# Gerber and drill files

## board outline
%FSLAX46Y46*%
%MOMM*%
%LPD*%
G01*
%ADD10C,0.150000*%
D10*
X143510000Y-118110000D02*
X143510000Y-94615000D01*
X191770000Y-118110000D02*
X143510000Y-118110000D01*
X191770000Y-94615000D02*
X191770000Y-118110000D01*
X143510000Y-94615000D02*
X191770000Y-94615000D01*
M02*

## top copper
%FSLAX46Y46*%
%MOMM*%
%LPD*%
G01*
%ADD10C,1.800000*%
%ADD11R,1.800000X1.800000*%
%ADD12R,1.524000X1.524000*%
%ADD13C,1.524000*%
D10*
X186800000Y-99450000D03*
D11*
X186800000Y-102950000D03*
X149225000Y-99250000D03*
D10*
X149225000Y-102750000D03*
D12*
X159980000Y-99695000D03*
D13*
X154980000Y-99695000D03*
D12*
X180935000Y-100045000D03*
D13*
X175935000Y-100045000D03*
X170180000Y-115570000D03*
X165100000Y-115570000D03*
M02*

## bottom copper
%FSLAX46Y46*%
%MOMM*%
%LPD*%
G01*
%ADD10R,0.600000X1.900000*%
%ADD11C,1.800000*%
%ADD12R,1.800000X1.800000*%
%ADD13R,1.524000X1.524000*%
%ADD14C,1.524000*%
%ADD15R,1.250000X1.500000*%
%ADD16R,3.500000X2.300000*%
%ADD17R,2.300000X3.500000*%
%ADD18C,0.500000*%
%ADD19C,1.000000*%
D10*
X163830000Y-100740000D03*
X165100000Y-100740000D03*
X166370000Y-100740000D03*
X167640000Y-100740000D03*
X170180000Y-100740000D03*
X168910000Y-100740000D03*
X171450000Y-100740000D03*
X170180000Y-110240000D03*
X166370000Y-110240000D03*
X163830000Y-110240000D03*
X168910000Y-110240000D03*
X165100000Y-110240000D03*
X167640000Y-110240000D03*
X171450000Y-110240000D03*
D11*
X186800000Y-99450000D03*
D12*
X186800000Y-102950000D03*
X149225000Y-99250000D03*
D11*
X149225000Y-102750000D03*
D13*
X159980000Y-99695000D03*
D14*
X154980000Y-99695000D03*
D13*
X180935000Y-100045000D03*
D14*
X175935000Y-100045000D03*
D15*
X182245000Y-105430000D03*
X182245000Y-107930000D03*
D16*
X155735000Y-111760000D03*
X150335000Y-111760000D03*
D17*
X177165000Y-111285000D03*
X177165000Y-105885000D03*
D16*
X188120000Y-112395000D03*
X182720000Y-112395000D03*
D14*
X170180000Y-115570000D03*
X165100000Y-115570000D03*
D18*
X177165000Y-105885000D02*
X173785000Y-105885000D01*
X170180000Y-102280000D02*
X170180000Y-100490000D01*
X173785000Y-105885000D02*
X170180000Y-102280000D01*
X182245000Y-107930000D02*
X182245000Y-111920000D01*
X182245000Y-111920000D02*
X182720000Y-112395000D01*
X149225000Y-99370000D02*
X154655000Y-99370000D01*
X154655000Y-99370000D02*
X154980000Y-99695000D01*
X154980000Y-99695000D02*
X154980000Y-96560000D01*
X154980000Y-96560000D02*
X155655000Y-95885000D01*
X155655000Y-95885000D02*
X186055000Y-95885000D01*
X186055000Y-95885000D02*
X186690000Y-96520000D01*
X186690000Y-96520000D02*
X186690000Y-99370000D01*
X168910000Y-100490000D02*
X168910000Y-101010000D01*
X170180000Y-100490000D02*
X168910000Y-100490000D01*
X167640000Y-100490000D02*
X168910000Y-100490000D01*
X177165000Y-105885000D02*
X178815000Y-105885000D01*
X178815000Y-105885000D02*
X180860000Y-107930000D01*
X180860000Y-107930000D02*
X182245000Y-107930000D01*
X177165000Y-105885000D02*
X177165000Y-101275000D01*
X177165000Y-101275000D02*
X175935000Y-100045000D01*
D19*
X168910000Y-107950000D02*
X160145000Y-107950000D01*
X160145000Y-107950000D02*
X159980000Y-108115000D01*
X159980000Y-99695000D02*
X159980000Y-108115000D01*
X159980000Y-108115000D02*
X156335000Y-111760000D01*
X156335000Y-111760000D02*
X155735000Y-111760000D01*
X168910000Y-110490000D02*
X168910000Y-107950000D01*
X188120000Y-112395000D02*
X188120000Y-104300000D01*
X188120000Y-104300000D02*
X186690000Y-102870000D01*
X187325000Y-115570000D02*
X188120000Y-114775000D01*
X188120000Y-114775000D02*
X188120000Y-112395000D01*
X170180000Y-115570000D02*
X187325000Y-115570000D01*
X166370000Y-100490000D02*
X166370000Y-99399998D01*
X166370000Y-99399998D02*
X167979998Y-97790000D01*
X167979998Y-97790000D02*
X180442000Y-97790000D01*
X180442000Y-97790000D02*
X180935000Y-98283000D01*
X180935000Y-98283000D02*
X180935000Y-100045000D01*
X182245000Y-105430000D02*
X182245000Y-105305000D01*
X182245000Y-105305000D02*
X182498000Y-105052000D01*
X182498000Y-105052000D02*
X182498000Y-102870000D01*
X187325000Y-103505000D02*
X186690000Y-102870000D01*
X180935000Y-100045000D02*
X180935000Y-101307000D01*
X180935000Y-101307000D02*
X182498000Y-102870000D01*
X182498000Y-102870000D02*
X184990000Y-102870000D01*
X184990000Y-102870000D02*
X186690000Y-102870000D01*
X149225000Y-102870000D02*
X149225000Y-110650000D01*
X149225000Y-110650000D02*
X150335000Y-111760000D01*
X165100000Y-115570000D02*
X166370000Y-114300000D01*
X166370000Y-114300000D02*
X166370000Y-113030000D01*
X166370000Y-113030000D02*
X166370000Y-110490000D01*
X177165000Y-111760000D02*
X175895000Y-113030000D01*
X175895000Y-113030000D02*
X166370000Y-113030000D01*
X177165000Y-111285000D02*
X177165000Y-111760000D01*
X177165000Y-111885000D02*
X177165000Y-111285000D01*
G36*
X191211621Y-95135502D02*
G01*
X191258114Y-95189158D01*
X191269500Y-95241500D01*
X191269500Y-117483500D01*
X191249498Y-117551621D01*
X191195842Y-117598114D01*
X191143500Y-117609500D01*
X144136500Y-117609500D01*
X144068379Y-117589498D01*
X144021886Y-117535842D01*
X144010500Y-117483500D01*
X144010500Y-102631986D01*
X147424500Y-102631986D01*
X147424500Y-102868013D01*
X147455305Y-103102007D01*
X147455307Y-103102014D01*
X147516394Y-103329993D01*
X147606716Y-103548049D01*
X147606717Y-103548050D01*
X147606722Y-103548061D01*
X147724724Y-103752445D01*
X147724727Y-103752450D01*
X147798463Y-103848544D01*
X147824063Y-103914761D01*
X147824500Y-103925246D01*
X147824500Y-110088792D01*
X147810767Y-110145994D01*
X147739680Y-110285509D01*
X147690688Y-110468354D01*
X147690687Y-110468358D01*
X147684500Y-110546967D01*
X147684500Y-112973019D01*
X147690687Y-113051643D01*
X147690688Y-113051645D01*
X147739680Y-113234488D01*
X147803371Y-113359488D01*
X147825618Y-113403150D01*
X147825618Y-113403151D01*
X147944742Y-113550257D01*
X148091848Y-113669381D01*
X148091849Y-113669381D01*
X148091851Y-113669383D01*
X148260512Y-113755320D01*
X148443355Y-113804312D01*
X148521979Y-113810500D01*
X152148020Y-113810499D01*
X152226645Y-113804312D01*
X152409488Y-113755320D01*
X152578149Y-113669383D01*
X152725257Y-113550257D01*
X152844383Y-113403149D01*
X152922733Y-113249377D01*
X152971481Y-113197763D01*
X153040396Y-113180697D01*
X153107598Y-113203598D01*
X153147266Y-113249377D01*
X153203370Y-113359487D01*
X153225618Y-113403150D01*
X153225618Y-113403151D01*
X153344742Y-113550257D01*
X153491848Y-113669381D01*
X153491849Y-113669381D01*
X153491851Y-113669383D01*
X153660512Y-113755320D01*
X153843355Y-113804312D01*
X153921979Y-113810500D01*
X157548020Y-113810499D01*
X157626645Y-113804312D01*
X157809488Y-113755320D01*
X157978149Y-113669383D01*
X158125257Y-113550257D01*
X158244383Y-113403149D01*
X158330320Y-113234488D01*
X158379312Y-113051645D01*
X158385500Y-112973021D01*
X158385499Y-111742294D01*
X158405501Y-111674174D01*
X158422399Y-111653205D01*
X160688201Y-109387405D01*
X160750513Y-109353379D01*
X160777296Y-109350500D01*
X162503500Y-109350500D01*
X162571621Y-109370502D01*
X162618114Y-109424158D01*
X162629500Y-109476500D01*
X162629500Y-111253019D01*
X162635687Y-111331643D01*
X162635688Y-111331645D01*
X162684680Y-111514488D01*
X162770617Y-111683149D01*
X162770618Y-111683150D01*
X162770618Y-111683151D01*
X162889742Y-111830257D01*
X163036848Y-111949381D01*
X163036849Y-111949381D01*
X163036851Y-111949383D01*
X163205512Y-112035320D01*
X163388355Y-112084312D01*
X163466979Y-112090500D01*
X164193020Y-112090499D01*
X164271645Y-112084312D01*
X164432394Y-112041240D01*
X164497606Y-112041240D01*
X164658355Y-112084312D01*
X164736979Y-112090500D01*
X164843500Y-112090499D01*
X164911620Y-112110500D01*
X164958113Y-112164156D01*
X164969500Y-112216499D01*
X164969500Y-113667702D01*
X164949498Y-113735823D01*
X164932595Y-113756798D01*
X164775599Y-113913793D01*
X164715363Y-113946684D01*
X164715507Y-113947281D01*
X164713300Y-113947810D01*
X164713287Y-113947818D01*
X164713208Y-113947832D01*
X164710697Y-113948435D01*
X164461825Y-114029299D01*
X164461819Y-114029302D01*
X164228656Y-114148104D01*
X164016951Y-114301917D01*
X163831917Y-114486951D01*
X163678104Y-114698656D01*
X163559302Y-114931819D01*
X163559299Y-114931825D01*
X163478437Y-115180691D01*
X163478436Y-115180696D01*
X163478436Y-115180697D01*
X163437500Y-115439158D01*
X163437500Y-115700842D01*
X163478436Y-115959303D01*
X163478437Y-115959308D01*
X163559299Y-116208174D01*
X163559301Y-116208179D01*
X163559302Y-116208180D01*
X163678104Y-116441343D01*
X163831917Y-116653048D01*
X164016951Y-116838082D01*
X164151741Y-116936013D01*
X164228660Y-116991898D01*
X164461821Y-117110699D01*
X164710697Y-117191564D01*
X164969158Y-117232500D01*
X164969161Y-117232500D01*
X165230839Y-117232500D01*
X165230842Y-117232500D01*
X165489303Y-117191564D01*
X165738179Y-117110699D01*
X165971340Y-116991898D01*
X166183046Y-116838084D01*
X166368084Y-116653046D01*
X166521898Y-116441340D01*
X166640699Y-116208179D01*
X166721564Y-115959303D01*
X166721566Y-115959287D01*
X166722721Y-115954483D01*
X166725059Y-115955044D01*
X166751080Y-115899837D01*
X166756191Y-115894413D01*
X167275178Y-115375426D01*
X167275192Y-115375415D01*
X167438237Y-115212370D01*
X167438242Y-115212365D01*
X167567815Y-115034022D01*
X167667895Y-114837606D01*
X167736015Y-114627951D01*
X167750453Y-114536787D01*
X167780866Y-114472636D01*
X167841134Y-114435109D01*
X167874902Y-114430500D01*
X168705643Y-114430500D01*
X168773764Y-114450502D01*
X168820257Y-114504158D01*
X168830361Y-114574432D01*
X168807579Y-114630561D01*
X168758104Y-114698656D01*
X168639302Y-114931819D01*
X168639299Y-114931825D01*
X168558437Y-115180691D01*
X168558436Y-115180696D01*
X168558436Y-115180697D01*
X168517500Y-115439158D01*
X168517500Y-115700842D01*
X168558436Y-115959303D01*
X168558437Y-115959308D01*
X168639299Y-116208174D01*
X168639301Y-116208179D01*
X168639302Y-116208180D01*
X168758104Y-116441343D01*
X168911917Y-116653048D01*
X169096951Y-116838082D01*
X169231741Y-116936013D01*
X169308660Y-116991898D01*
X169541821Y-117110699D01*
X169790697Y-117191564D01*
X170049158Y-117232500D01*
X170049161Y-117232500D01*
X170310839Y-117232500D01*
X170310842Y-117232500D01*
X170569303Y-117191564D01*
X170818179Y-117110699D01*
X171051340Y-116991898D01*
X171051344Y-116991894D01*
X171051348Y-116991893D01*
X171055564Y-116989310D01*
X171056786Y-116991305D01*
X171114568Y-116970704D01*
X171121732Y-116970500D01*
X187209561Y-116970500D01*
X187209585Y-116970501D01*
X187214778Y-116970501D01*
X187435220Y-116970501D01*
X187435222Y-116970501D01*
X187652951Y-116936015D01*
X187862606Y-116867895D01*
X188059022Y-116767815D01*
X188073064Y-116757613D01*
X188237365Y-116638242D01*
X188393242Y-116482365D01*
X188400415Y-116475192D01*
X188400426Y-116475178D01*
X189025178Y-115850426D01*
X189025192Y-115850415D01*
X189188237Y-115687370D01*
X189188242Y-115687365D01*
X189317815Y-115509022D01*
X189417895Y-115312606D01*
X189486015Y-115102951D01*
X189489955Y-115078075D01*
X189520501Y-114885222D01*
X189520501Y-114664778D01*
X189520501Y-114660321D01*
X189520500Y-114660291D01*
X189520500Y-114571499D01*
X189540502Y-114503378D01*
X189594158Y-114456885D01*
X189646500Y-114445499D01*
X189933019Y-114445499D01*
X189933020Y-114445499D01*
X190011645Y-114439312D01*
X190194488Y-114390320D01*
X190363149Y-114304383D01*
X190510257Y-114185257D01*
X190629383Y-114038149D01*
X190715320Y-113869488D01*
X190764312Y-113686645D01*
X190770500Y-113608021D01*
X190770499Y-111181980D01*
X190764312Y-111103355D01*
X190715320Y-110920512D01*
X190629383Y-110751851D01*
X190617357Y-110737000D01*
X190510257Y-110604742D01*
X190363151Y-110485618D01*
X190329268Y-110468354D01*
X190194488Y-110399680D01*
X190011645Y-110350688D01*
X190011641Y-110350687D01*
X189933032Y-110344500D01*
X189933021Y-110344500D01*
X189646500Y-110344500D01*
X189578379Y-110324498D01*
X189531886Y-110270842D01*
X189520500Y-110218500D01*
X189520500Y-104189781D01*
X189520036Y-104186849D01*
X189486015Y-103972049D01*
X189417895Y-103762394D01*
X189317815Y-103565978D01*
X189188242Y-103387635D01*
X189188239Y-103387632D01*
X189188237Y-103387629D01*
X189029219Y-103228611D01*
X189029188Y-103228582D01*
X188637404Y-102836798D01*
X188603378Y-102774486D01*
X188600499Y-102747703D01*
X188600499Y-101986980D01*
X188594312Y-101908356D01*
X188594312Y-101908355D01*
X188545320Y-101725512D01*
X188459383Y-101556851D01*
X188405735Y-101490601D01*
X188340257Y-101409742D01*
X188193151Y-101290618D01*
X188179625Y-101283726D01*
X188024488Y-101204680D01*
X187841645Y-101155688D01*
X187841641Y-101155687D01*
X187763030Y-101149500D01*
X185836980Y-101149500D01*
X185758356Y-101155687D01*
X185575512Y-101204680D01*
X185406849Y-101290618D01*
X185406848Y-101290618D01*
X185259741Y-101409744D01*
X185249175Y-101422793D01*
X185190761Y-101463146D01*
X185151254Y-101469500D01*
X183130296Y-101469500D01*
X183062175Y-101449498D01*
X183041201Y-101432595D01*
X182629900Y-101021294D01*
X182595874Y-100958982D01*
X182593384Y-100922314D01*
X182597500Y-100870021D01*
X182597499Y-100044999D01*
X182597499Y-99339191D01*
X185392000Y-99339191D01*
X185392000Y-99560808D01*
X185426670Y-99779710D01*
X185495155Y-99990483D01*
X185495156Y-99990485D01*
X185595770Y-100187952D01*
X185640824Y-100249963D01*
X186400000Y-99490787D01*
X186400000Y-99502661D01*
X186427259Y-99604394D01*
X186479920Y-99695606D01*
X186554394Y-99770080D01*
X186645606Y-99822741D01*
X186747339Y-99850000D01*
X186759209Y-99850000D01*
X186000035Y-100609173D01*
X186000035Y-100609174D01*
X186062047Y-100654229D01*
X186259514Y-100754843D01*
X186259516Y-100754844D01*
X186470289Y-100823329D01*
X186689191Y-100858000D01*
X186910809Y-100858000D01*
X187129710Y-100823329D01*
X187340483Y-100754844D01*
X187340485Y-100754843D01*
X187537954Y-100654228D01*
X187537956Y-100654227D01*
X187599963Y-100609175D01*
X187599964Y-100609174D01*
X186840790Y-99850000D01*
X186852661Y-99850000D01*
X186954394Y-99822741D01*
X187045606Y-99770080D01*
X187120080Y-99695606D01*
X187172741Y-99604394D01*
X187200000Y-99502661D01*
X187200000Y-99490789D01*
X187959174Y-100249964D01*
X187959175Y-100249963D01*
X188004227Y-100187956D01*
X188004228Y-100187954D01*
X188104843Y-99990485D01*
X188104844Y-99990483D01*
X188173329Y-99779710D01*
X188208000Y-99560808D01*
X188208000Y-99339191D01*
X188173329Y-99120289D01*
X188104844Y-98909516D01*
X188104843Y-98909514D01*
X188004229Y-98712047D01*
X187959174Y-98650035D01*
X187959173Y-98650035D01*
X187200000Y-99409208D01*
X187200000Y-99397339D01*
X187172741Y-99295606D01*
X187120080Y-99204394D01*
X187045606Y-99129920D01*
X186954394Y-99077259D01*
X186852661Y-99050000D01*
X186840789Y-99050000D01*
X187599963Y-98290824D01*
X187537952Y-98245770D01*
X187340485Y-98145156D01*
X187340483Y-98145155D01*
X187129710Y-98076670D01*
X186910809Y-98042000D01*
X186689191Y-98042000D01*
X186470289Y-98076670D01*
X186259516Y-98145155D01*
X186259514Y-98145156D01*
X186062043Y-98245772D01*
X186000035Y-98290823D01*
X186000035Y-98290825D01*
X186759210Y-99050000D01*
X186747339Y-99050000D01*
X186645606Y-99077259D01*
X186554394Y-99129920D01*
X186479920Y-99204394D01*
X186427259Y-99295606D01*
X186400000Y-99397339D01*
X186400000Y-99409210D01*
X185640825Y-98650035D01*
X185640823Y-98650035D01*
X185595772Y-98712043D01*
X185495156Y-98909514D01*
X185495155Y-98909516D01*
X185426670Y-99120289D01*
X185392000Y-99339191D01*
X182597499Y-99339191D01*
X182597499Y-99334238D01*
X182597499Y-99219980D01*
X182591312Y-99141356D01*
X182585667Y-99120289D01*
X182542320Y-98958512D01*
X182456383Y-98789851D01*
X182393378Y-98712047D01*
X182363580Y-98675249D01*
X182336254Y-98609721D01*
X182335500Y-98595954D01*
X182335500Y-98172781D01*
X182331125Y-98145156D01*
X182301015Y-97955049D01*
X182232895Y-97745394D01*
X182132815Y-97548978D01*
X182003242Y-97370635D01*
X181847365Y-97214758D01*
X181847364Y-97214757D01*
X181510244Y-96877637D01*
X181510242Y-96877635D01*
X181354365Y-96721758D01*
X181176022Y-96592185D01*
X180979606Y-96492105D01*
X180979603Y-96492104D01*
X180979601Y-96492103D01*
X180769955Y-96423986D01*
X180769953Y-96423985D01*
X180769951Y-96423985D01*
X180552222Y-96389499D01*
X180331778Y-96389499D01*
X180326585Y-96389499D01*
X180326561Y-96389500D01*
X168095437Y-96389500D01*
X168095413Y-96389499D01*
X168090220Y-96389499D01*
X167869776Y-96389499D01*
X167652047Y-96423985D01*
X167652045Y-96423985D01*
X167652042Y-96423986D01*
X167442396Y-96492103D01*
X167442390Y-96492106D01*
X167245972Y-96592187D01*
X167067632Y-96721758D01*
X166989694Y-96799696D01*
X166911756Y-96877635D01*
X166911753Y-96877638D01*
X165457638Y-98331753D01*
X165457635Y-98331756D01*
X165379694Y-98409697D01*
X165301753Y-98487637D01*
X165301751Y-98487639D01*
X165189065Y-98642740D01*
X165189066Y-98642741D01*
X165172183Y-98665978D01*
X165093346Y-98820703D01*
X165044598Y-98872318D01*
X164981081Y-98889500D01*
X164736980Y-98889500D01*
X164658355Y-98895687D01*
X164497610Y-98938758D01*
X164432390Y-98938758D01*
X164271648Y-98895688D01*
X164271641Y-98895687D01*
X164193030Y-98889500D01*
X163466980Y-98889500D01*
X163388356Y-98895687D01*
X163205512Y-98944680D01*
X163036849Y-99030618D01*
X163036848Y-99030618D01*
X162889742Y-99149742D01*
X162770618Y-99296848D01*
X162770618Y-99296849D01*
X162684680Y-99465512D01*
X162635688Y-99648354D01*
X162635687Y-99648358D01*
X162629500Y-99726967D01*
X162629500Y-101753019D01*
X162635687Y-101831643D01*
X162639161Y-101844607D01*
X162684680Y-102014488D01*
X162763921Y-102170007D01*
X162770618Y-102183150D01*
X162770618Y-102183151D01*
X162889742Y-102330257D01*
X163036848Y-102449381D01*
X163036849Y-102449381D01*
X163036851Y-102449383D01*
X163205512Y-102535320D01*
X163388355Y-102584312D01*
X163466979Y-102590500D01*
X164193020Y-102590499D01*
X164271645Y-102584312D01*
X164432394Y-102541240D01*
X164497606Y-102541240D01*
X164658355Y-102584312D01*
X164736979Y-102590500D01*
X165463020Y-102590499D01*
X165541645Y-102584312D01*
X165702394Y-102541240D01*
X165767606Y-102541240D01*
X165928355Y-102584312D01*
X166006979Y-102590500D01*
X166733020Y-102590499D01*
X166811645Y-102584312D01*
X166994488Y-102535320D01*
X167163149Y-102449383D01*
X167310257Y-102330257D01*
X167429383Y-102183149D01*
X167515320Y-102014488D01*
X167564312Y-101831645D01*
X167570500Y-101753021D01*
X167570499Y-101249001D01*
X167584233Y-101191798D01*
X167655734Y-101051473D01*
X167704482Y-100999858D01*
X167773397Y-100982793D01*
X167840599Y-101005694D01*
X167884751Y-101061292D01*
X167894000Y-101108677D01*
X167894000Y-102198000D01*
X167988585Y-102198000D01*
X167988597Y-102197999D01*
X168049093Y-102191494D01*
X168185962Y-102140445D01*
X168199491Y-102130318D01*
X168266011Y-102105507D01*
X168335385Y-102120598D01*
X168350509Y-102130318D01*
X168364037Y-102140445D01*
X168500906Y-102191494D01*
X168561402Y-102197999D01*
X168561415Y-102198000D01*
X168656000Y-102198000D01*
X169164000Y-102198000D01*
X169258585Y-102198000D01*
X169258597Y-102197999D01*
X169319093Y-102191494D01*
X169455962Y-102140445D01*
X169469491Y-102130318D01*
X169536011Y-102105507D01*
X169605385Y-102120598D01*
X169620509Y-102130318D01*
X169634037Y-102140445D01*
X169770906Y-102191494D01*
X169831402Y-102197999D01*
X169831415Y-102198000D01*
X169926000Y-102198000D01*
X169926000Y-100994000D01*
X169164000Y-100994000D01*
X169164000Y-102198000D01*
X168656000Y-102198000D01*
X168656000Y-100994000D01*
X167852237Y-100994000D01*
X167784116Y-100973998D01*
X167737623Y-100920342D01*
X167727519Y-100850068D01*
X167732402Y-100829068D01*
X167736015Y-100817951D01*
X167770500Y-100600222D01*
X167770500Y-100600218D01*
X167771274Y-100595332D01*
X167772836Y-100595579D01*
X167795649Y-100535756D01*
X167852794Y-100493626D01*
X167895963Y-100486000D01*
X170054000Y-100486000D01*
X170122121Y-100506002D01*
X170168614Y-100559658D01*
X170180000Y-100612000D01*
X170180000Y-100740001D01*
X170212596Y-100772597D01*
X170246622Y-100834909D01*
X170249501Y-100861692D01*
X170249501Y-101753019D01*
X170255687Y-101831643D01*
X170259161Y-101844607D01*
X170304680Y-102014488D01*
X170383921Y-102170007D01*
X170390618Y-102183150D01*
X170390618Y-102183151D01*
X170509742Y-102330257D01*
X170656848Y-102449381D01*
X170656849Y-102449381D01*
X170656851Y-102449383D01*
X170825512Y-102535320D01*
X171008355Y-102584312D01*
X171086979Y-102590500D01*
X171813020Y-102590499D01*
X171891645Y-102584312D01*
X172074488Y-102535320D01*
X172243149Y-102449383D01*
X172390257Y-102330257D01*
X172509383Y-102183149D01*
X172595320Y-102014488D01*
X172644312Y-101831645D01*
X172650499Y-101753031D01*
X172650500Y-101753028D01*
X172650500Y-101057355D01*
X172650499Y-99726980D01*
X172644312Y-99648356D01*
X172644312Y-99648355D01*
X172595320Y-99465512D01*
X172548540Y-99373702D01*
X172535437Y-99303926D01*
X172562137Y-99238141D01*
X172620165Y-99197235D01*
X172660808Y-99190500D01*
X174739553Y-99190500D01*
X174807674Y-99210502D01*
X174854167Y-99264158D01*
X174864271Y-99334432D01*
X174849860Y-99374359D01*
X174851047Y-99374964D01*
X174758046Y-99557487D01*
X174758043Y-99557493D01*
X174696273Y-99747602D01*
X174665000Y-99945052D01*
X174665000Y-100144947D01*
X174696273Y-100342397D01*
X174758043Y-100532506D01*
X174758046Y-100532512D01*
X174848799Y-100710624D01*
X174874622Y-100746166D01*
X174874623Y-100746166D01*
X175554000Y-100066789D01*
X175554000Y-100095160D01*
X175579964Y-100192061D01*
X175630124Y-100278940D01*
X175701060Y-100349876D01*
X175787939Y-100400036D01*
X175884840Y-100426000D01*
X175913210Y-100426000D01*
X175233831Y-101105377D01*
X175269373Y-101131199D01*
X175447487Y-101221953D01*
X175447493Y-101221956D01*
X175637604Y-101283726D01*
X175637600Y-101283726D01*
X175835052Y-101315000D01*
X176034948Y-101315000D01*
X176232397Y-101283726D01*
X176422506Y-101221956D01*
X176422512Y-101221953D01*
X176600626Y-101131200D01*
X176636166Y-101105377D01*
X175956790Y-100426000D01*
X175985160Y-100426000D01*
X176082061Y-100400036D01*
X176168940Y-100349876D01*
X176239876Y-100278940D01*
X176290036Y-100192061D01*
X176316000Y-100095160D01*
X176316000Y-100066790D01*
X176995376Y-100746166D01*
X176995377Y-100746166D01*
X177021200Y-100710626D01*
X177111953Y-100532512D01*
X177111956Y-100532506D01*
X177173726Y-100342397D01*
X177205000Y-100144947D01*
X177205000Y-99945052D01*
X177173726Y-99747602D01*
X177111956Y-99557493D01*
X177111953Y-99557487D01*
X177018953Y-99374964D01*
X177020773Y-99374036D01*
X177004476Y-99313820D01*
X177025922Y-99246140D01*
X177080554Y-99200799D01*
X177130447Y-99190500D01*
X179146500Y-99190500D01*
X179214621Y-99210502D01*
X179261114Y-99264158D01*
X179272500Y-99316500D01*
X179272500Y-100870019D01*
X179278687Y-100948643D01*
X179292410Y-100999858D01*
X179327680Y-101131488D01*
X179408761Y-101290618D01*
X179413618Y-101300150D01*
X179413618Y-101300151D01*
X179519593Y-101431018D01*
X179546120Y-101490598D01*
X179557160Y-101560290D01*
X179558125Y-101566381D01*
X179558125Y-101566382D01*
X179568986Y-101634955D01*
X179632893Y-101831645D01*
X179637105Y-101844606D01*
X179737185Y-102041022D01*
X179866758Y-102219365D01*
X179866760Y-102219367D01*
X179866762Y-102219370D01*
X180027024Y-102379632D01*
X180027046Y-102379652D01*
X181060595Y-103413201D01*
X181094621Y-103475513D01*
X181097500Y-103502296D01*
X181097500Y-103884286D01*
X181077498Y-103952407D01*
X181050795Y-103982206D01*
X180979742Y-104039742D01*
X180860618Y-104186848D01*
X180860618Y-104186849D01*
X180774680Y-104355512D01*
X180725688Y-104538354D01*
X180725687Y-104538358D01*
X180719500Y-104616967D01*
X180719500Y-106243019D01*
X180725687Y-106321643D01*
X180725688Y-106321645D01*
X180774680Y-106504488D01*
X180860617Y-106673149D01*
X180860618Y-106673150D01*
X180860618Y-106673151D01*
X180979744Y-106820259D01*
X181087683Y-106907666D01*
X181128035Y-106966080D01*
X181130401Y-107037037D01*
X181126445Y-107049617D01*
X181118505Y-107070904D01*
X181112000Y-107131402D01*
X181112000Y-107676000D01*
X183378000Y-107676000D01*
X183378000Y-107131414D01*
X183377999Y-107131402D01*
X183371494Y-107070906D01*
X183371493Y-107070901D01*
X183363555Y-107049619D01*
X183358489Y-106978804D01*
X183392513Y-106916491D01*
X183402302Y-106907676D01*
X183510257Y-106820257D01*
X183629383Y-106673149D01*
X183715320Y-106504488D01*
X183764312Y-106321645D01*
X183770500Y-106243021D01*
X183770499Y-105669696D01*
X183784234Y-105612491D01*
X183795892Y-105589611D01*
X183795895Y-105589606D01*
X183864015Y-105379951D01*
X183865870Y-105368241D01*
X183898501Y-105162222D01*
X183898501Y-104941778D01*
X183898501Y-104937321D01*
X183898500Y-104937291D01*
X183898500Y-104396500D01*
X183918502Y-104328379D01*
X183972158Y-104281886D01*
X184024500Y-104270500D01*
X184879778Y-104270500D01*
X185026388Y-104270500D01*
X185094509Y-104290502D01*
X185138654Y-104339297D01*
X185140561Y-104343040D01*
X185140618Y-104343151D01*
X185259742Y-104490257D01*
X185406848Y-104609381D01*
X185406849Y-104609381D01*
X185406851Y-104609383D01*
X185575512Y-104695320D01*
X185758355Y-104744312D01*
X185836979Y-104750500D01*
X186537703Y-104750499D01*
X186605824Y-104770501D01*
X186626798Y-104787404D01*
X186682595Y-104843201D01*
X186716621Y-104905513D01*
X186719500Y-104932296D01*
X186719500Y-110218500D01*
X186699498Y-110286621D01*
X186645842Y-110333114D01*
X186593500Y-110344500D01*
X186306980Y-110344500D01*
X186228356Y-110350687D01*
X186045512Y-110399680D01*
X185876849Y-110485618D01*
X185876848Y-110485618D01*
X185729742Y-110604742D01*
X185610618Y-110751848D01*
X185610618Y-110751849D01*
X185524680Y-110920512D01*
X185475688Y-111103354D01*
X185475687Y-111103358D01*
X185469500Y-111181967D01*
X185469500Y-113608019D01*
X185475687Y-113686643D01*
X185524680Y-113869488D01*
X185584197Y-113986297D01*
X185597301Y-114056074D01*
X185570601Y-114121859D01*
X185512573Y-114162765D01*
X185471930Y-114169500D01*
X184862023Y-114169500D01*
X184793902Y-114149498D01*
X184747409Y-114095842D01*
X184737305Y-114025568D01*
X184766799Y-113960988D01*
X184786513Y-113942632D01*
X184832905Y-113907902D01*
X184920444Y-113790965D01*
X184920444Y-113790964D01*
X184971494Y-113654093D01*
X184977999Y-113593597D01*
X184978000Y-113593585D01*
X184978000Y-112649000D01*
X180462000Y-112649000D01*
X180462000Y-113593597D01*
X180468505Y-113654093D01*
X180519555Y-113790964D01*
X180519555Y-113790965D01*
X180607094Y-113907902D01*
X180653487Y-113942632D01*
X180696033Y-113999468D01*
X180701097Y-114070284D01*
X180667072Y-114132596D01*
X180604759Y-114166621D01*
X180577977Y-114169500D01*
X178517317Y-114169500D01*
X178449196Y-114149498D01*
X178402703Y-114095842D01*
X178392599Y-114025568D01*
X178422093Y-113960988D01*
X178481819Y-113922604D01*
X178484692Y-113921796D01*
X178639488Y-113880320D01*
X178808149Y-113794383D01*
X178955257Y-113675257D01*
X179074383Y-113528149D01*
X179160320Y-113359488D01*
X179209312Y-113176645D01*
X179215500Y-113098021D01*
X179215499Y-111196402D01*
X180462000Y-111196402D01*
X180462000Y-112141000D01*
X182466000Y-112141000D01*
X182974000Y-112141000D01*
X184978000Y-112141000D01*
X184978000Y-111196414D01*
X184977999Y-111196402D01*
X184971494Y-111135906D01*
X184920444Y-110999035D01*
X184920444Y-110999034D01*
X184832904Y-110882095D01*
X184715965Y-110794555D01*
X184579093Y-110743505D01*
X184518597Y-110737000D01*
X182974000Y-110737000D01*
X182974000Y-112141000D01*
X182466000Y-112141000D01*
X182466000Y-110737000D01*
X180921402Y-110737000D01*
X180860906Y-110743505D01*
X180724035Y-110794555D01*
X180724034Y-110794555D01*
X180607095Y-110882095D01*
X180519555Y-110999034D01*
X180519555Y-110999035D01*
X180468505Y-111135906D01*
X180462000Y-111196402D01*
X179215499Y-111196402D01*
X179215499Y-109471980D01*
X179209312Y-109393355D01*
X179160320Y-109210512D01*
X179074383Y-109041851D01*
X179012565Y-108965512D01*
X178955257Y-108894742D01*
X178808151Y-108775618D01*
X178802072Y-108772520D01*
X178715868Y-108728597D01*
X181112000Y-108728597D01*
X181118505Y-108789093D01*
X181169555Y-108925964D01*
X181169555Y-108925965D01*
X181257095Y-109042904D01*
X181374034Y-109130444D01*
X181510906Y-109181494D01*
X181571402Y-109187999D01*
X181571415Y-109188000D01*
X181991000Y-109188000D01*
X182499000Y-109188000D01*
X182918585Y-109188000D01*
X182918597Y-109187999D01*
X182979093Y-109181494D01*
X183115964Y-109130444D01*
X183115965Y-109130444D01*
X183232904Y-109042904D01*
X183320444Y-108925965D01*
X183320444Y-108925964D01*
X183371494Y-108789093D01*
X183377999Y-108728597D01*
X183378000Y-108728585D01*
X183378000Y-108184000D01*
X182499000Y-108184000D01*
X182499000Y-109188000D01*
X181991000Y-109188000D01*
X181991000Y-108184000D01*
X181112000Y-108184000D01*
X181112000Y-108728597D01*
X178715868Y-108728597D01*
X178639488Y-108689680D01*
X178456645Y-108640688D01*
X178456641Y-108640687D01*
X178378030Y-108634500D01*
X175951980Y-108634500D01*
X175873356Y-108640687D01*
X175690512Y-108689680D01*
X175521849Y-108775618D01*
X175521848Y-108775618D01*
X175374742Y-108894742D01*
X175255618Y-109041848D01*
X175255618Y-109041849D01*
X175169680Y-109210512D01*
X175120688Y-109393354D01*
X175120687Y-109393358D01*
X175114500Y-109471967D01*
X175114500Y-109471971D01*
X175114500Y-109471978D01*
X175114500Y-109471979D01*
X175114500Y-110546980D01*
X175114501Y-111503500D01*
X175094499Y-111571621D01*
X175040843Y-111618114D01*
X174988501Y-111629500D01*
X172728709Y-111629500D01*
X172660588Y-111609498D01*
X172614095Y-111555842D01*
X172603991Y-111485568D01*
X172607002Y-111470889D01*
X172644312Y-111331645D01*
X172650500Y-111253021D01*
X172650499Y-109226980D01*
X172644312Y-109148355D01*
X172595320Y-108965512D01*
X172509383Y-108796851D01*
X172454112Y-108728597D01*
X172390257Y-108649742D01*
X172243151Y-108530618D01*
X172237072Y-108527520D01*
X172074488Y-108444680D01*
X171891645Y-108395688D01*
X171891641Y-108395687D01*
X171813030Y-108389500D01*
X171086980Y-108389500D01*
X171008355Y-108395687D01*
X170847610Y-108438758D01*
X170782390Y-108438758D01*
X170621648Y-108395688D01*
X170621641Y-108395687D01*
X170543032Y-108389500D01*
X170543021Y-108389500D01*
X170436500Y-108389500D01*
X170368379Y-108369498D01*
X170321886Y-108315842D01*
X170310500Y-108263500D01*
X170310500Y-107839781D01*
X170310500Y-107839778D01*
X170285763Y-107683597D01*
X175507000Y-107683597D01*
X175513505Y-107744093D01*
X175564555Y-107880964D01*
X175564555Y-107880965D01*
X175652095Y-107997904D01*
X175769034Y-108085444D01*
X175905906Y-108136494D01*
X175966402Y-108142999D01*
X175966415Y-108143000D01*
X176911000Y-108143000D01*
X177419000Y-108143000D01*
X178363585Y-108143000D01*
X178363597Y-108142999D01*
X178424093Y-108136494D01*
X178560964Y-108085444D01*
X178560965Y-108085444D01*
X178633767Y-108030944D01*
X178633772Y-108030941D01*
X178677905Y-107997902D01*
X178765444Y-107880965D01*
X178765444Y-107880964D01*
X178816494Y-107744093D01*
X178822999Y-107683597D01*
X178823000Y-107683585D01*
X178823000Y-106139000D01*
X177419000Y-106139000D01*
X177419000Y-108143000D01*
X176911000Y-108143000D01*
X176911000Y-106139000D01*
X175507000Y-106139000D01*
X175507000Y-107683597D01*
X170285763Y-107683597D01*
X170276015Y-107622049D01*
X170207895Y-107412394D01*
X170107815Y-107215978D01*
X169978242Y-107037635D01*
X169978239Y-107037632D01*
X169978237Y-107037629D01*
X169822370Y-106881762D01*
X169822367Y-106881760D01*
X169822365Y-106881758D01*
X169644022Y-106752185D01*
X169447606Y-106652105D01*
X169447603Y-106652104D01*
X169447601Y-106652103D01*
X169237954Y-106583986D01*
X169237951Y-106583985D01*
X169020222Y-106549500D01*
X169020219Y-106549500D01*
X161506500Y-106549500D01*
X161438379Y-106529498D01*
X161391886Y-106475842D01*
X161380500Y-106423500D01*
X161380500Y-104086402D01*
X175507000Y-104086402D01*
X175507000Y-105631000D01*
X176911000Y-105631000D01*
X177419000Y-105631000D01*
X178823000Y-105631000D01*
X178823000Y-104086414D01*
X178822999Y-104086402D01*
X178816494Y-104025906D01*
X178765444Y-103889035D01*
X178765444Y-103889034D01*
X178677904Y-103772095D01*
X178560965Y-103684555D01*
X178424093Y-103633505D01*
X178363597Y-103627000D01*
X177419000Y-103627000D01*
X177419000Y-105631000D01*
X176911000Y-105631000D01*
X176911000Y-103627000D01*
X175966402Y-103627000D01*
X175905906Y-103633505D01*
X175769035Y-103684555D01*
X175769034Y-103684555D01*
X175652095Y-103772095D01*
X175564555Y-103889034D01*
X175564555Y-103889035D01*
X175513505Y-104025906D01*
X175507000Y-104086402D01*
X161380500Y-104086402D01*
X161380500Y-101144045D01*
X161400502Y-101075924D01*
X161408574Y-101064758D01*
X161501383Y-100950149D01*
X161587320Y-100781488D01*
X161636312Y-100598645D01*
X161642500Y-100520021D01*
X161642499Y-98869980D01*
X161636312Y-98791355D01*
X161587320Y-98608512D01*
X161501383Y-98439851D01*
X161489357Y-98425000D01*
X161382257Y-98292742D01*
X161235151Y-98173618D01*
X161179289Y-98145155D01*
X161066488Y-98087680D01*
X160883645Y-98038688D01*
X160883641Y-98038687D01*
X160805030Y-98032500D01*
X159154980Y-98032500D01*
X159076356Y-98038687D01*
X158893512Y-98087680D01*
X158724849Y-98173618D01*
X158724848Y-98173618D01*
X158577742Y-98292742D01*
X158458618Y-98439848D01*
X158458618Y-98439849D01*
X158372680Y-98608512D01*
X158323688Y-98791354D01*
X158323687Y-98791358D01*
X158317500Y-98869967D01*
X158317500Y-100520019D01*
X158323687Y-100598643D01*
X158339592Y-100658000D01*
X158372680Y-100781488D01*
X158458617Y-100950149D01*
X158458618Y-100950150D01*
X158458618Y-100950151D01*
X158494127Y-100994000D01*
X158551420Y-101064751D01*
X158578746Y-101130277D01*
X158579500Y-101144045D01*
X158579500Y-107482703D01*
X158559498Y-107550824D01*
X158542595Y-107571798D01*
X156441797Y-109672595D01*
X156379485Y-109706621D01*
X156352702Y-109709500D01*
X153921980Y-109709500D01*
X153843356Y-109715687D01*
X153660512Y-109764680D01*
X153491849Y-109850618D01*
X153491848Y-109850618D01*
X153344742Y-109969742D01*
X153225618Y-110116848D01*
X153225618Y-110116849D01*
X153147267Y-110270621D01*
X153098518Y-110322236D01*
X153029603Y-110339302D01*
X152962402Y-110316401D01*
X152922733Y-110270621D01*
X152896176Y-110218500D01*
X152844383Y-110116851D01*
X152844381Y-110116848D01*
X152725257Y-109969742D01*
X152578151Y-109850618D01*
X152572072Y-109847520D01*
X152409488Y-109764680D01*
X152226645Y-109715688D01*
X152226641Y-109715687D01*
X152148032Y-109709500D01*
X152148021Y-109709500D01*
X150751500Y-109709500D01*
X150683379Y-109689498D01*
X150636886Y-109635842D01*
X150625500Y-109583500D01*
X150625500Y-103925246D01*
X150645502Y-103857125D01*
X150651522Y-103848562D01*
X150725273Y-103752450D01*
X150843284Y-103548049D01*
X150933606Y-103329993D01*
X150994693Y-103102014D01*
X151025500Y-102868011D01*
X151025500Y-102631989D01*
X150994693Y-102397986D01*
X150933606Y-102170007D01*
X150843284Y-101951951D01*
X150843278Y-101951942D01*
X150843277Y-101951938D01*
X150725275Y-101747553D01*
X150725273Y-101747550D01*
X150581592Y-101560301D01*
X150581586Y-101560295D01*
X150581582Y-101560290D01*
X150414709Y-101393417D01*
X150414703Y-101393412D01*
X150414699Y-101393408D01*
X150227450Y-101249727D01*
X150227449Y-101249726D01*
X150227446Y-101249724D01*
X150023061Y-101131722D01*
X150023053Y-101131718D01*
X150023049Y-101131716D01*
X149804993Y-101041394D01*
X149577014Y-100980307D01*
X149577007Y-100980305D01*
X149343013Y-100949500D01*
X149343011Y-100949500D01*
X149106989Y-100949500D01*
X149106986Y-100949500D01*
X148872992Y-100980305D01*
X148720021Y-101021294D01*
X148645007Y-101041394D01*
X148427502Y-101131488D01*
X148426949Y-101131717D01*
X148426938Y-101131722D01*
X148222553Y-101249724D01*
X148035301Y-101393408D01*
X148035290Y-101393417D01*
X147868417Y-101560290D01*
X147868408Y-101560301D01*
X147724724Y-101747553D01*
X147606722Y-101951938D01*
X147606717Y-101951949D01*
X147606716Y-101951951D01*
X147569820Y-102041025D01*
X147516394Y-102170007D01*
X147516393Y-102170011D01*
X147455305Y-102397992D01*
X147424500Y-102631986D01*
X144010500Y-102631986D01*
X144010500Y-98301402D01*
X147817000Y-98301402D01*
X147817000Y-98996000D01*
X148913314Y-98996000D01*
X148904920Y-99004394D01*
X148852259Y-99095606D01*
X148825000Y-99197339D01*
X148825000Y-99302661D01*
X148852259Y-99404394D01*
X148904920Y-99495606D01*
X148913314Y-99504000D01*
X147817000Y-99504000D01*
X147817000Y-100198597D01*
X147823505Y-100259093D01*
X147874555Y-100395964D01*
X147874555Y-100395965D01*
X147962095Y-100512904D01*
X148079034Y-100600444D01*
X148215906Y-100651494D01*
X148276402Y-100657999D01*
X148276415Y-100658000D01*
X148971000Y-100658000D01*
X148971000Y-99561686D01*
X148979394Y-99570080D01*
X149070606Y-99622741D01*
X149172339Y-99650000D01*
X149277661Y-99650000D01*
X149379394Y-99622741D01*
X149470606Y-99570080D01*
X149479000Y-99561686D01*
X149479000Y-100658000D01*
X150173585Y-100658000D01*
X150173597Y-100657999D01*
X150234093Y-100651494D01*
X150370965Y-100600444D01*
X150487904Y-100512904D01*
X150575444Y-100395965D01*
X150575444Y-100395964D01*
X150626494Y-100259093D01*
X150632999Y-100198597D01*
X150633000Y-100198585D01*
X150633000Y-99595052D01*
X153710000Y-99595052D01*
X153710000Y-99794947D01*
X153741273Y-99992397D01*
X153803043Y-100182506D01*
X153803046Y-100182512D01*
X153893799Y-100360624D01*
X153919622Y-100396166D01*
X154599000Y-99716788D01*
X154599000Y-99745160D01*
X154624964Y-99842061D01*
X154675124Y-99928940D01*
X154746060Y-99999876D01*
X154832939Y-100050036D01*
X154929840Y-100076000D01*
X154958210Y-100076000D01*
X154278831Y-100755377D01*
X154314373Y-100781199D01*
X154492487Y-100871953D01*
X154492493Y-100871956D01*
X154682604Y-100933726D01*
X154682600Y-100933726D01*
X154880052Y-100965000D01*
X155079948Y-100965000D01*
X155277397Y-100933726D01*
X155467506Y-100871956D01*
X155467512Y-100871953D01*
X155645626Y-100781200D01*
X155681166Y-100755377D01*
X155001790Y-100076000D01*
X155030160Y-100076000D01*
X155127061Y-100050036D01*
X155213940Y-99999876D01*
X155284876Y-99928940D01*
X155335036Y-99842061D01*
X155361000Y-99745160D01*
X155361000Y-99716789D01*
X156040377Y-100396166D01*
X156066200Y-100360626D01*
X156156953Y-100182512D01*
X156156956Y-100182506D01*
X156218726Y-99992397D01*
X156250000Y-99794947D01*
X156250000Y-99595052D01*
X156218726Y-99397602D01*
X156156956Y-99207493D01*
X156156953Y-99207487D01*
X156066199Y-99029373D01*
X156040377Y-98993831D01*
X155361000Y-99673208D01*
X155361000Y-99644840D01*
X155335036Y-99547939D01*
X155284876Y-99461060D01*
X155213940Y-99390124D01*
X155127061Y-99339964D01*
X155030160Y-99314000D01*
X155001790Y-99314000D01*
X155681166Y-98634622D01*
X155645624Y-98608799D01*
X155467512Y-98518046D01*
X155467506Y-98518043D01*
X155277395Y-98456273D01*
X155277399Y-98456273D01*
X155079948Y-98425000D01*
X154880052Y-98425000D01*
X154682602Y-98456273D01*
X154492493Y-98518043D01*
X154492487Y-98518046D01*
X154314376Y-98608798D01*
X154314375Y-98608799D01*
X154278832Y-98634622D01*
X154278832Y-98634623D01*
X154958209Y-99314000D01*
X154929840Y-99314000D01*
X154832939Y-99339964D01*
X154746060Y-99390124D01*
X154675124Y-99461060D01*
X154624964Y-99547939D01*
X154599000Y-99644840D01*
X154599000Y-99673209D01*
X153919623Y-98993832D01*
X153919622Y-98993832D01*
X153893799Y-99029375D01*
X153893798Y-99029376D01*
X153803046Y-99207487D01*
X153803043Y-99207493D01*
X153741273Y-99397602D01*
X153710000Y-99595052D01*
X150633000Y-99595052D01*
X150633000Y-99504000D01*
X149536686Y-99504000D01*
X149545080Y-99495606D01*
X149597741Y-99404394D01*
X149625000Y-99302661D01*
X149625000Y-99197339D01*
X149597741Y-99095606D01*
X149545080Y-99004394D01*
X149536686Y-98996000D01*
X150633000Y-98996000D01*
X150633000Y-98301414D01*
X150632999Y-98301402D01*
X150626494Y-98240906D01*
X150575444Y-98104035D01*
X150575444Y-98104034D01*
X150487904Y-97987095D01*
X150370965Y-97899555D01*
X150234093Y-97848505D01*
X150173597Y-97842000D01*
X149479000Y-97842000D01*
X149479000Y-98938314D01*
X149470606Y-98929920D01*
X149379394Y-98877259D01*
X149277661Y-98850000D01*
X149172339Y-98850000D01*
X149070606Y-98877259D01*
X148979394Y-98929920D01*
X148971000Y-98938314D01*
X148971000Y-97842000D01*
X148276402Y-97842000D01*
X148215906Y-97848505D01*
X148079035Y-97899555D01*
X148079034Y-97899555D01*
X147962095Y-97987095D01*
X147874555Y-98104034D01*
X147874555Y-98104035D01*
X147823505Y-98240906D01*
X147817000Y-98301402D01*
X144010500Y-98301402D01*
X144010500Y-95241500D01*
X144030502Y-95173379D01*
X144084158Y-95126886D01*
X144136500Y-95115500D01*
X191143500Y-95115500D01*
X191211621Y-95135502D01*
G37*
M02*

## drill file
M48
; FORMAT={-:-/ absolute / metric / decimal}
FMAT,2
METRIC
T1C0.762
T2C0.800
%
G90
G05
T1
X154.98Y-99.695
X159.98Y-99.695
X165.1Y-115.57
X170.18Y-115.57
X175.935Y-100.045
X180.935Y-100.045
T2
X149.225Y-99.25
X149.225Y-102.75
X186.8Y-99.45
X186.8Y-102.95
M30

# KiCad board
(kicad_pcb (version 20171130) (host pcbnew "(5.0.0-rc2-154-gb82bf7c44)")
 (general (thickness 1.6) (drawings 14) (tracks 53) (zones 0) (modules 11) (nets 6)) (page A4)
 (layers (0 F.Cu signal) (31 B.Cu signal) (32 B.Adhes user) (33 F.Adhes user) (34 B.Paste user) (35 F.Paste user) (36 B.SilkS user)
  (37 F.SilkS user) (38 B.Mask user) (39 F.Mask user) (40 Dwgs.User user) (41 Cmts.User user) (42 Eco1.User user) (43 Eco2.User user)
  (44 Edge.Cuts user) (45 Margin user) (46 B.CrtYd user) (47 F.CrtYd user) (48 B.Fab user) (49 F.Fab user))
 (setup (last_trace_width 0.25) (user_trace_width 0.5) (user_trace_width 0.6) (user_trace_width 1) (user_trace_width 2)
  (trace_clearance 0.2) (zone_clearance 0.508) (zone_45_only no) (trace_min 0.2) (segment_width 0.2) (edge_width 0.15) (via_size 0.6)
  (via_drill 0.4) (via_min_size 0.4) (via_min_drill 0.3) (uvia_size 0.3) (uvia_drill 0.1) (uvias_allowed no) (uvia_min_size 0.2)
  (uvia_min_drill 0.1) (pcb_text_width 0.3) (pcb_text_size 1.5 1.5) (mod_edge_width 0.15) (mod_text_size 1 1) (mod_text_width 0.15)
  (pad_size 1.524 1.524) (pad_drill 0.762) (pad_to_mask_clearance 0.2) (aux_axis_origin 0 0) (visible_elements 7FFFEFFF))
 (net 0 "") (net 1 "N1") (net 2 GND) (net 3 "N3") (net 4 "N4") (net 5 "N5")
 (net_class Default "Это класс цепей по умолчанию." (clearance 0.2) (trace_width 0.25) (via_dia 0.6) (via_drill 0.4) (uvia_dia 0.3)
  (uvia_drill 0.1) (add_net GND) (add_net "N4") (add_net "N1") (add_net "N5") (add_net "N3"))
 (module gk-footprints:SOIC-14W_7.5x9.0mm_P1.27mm (layer B.Cu) (at 167.64 105.49 270)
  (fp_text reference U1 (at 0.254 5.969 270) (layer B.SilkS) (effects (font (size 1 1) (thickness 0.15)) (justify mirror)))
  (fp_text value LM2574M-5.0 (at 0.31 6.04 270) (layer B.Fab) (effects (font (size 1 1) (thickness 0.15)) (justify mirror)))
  (pad 1 smd rect (at -4.75 3.81 270) (size 1.9 0.6) (layers B.Cu B.Paste B.Mask))
  (pad 2 smd rect (at -4.75 2.54 270) (size 1.9 0.6) (layers B.Cu B.Paste B.Mask))
  (pad 3 smd rect (at -4.75 1.27 270) (size 1.9 0.6) (layers B.Cu B.Paste B.Mask) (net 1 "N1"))
  (pad 4 smd rect (at -4.75 0 270) (size 1.9 0.6) (layers B.Cu B.Paste B.Mask) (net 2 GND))
  (pad 6 smd rect (at -4.75 -2.54 270) (size 1.9 0.6) (layers B.Cu B.Paste B.Mask) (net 2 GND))
  (pad 5 smd rect (at -4.75 -1.27 270) (size 1.9 0.6) (layers B.Cu B.Paste B.Mask) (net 2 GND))
  (pad 7 smd rect (at -4.75 -3.81 270) (size 1.9 0.6) (layers B.Cu B.Paste B.Mask))
  (pad 9 smd rect (at 4.75 -2.54 270) (size 1.9 0.6) (layers B.Cu B.Paste B.Mask))
  (pad 12 smd rect (at 4.75 1.27 270) (size 1.9 0.6) (layers B.Cu B.Paste B.Mask) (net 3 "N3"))
  (pad 14 smd rect (at 4.75 3.81 270) (size 1.9 0.6) (layers B.Cu B.Paste B.Mask))
  (pad 10 smd rect (at 4.75 -1.27 270) (size 1.9 0.6) (layers B.Cu B.Paste B.Mask) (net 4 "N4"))
  (pad 13 smd rect (at 4.75 2.54 270) (size 1.9 0.6) (layers B.Cu B.Paste B.Mask))
  (pad 11 smd rect (at 4.75 0 270) (size 1.9 0.6) (layers B.Cu B.Paste B.Mask))
  (pad 8 smd rect (at 4.75 -3.81 270) (size 1.9 0.6) (layers B.Cu B.Paste B.Mask)))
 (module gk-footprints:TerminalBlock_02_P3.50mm (layer F.Cu) (at 186.8 101.2 90)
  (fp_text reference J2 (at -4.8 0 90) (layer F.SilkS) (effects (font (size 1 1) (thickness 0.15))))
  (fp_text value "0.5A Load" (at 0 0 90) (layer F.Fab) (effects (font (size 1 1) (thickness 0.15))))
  (pad 2 thru_hole circle (at 1.75 0 90) (size 1.8 1.8) (drill 0.8) (layers *.Cu *.Mask) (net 2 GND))
  (pad 1 thru_hole rect (at -1.75 0 90) (size 1.8 1.8) (drill 0.8) (layers *.Cu *.Mask) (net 1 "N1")))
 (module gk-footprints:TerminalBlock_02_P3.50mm (layer F.Cu) (at 149.225 101 270)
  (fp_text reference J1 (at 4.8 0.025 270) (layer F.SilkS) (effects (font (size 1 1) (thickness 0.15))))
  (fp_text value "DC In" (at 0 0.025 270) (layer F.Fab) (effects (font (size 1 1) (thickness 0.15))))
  (pad 1 thru_hole rect (at -1.75 0 270) (size 1.8 1.8) (drill 0.8) (layers *.Cu *.Mask) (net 2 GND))
  (pad 2 thru_hole circle (at 1.75 0 270) (size 1.8 1.8) (drill 0.8) (layers *.Cu *.Mask) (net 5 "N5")))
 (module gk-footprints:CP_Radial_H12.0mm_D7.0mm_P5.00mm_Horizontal (layer F.Cu) (at 157.48 105.695 180)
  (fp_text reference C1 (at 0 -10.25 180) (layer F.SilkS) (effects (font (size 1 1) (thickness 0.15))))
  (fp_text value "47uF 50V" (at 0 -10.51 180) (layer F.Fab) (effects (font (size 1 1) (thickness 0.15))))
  (pad 1 thru_hole rect (at -2.5 6 180) (size 1.524 1.524) (drill 0.762) (layers *.Cu *.Mask) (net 4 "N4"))
  (pad 2 thru_hole circle (at 2.5 6 180) (size 1.524 1.524) (drill 0.762) (layers *.Cu *.Mask) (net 2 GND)))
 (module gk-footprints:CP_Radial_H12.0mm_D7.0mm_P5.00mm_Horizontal (layer F.Cu) (at 178.435 106.045 180)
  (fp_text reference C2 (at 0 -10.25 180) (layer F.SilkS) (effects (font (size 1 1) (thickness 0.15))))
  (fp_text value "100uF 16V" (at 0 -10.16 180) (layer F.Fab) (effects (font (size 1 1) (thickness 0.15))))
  (pad 1 thru_hole rect (at -2.5 6 180) (size 1.524 1.524) (drill 0.762) (layers *.Cu *.Mask) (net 1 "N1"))
  (pad 2 thru_hole circle (at 2.5 6 180) (size 1.524 1.524) (drill 0.762) (layers *.Cu *.Mask) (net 2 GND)))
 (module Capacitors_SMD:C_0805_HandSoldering (layer B.Cu) (at 182.245 106.68 270)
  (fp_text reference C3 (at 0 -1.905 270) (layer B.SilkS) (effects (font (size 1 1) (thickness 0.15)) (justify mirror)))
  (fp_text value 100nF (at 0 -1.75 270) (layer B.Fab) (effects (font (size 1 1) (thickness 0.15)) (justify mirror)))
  (pad 1 smd rect (at -1.25 0 270) (size 1.5 1.25) (layers B.Cu B.Paste B.Mask) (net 1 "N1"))
  (pad 2 smd rect (at 1.25 0 270) (size 1.5 1.25) (layers B.Cu B.Paste B.Mask) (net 2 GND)))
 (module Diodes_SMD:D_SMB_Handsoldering (layer B.Cu) (at 153.035 111.76 180)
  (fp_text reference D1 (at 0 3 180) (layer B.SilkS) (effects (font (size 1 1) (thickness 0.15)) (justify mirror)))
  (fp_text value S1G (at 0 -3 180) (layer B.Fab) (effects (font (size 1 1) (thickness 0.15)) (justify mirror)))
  (pad 1 smd rect (at -2.7 0 180) (size 3.5 2.3) (layers B.Cu B.Paste B.Mask) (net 4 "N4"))
  (pad 2 smd rect (at 2.7 0 180) (size 3.5 2.3) (layers B.Cu B.Paste B.Mask) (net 5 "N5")))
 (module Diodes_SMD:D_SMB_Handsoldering (layer B.Cu) (at 177.165 108.585 90)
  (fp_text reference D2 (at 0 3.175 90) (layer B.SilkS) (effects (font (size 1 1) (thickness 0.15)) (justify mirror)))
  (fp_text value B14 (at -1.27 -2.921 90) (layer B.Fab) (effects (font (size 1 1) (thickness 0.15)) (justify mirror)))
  (pad 1 smd rect (at -2.7 0 90) (size 3.5 2.3) (layers B.Cu B.Paste B.Mask) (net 3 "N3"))
  (pad 2 smd rect (at 2.7 0 90) (size 3.5 2.3) (layers B.Cu B.Paste B.Mask) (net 2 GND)))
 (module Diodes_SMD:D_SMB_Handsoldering (layer B.Cu) (at 185.42 112.395 180)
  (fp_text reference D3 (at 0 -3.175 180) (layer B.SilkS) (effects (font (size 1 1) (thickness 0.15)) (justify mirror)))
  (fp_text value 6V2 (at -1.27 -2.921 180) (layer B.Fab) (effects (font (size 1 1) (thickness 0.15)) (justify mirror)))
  (pad 1 smd rect (at -2.7 0 180) (size 3.5 2.3) (layers B.Cu B.Paste B.Mask) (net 1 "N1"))
  (pad 2 smd rect (at 2.7 0 180) (size 3.5 2.3) (layers B.Cu B.Paste B.Mask) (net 2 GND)))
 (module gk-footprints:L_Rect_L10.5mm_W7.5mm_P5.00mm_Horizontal (layer F.Cu) (at 167.64 108.57)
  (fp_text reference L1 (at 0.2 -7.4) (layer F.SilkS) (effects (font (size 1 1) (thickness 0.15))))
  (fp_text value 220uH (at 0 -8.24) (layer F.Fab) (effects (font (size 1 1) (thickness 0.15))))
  (pad 1 thru_hole circle (at 2.54 7) (size 1.524 1.524) (drill 0.762) (layers *.Cu *.Mask) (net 1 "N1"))
  (pad 2 thru_hole circle (at -2.54 7) (size 1.524 1.524) (drill 0.762) (layers *.Cu *.Mask) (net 3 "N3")))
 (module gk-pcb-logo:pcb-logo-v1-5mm (layer F.Cu) (at 149.225 111.125 270)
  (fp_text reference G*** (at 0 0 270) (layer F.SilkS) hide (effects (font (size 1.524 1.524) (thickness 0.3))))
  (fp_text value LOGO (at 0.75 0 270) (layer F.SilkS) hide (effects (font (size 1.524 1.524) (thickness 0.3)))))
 (gr_line (start 143.51 118.11) (end 143.51 94.615) (layer Edge.Cuts) (width 0.15))
 (gr_line (start 191.77 118.11) (end 143.51 118.11) (layer Edge.Cuts) (width 0.15))
 (gr_line (start 191.77 94.615) (end 191.77 118.11) (layer Edge.Cuts) (width 0.15))
 (gr_line (start 143.51 94.615) (end 191.77 94.615) (layer Edge.Cuts) (width 0.15))
 (segment (start 177.165 105.885) (end 173.785 105.885) (width 0.5) (layer B.Cu) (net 2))
 (segment (start 170.18 102.28) (end 170.18 100.49) (width 0.5) (layer B.Cu) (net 2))
 (segment (start 173.785 105.885) (end 170.18 102.28) (width 0.5) (layer B.Cu) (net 2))
 (segment (start 182.245 107.93) (end 182.245 111.92) (width 0.5) (layer B.Cu) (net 2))
 (segment (start 182.245 111.92) (end 182.72 112.395) (width 0.5) (layer B.Cu) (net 2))
 (segment (start 149.225 99.37) (end 154.655 99.37) (width 0.5) (layer B.Cu) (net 2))
 (segment (start 154.655 99.37) (end 154.98 99.695) (width 0.5) (layer B.Cu) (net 2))
 (segment (start 154.98 99.695) (end 154.98 96.56) (width 0.5) (layer B.Cu) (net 2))
 (segment (start 154.98 96.56) (end 155.655 95.885) (width 0.5) (layer B.Cu) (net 2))
 (segment (start 155.655 95.885) (end 186.055 95.885) (width 0.5) (layer B.Cu) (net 2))
 (segment (start 186.055 95.885) (end 186.69 96.52) (width 0.5) (layer B.Cu) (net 2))
 (segment (start 186.69 96.52) (end 186.69 99.37) (width 0.5) (layer B.Cu) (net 2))
 (segment (start 168.91 100.49) (end 168.91 101.01) (width 0.5) (layer B.Cu) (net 2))
 (segment (start 170.18 100.49) (end 168.91 100.49) (width 0.5) (layer B.Cu) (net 2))
 (segment (start 167.64 100.49) (end 168.91 100.49) (width 0.5) (layer B.Cu) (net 2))
 (segment (start 177.165 105.885) (end 178.815 105.885) (width 0.5) (layer B.Cu) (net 2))
 (segment (start 178.815 105.885) (end 180.86 107.93) (width 0.5) (layer B.Cu) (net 2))
 (segment (start 180.86 107.93) (end 182.245 107.93) (width 0.5) (layer B.Cu) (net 2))
 (segment (start 177.165 105.885) (end 177.165 101.275) (width 0.5) (layer B.Cu) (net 2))
 (segment (start 177.165 101.275) (end 175.935 100.045) (width 0.5) (layer B.Cu) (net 2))
 (segment (start 168.91 107.95) (end 160.145 107.95) (width 1) (layer B.Cu) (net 4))
 (segment (start 160.145 107.95) (end 159.98 108.115) (width 1) (layer B.Cu) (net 4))
 (segment (start 159.98 99.695) (end 159.98 108.115) (width 1) (layer B.Cu) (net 4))
 (segment (start 159.98 108.115) (end 156.335 111.76) (width 1) (layer B.Cu) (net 4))
 (segment (start 156.335 111.76) (end 155.735 111.76) (width 1) (layer B.Cu) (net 4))
 (segment (start 168.91 110.49) (end 168.91 107.95) (width 1) (layer B.Cu) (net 4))
 (segment (start 188.12 112.395) (end 188.12 104.3) (width 1) (layer B.Cu) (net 1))
 (segment (start 188.12 104.3) (end 186.69 102.87) (width 1) (layer B.Cu) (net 1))
 (segment (start 187.325 115.57) (end 188.12 114.775) (width 1) (layer B.Cu) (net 1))
 (segment (start 188.12 114.775) (end 188.12 112.395) (width 1) (layer B.Cu) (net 1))
 (segment (start 170.18 115.57) (end 187.325 115.57) (width 1) (layer B.Cu) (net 1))
 (segment (start 166.37 100.49) (end 166.37 99.399998) (width 1) (layer B.Cu) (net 1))
 (segment (start 166.37 99.399998) (end 167.979998 97.79) (width 1) (layer B.Cu) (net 1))
 (segment (start 167.979998 97.79) (end 180.442 97.79) (width 1) (layer B.Cu) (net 1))
 (segment (start 180.442 97.79) (end 180.935 98.283) (width 1) (layer B.Cu) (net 1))
 (segment (start 180.935 98.283) (end 180.935 100.045) (width 1) (layer B.Cu) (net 1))
 (segment (start 182.245 105.43) (end 182.245 105.305) (width 1) (layer B.Cu) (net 1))
 (segment (start 182.245 105.305) (end 182.498 105.052) (width 1) (layer B.Cu) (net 1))
 (segment (start 182.498 105.052) (end 182.498 102.87) (width 1) (layer B.Cu) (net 1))
 (segment (start 187.325 103.505) (end 186.69 102.87) (width 1) (layer B.Cu) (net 1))
 (segment (start 180.935 100.045) (end 180.935 101.307) (width 1) (layer B.Cu) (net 1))
 (segment (start 180.935 101.307) (end 182.498 102.87) (width 1) (layer B.Cu) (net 1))
 (segment (start 182.498 102.87) (end 184.99 102.87) (width 1) (layer B.Cu) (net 1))
 (segment (start 184.99 102.87) (end 186.69 102.87) (width 1) (layer B.Cu) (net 1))
 (segment (start 149.225 102.87) (end 149.225 110.65) (width 1) (layer B.Cu) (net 5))
 (segment (start 149.225 110.65) (end 150.335 111.76) (width 1) (layer B.Cu) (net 5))
 (segment (start 165.1 115.57) (end 166.37 114.3) (width 1) (layer B.Cu) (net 3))
 (segment (start 166.37 114.3) (end 166.37 113.03) (width 1) (layer B.Cu) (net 3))
 (segment (start 166.37 113.03) (end 166.37 110.49) (width 1) (layer B.Cu) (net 3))
 (segment (start 177.165 111.76) (end 175.895 113.03) (width 1) (layer B.Cu) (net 3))
 (segment (start 175.895 113.03) (end 166.37 113.03) (width 1) (layer B.Cu) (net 3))
 (segment (start 177.165 111.285) (end 177.165 111.76) (width 1) (layer B.Cu) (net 3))
 (segment (start 177.165 111.885) (end 177.165 111.285) (width 1) (layer B.Cu) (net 3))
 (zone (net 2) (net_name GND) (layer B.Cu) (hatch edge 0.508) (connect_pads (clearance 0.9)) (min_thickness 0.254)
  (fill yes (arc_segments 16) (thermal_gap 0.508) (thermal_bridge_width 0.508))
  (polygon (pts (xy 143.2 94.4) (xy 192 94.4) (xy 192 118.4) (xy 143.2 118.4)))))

